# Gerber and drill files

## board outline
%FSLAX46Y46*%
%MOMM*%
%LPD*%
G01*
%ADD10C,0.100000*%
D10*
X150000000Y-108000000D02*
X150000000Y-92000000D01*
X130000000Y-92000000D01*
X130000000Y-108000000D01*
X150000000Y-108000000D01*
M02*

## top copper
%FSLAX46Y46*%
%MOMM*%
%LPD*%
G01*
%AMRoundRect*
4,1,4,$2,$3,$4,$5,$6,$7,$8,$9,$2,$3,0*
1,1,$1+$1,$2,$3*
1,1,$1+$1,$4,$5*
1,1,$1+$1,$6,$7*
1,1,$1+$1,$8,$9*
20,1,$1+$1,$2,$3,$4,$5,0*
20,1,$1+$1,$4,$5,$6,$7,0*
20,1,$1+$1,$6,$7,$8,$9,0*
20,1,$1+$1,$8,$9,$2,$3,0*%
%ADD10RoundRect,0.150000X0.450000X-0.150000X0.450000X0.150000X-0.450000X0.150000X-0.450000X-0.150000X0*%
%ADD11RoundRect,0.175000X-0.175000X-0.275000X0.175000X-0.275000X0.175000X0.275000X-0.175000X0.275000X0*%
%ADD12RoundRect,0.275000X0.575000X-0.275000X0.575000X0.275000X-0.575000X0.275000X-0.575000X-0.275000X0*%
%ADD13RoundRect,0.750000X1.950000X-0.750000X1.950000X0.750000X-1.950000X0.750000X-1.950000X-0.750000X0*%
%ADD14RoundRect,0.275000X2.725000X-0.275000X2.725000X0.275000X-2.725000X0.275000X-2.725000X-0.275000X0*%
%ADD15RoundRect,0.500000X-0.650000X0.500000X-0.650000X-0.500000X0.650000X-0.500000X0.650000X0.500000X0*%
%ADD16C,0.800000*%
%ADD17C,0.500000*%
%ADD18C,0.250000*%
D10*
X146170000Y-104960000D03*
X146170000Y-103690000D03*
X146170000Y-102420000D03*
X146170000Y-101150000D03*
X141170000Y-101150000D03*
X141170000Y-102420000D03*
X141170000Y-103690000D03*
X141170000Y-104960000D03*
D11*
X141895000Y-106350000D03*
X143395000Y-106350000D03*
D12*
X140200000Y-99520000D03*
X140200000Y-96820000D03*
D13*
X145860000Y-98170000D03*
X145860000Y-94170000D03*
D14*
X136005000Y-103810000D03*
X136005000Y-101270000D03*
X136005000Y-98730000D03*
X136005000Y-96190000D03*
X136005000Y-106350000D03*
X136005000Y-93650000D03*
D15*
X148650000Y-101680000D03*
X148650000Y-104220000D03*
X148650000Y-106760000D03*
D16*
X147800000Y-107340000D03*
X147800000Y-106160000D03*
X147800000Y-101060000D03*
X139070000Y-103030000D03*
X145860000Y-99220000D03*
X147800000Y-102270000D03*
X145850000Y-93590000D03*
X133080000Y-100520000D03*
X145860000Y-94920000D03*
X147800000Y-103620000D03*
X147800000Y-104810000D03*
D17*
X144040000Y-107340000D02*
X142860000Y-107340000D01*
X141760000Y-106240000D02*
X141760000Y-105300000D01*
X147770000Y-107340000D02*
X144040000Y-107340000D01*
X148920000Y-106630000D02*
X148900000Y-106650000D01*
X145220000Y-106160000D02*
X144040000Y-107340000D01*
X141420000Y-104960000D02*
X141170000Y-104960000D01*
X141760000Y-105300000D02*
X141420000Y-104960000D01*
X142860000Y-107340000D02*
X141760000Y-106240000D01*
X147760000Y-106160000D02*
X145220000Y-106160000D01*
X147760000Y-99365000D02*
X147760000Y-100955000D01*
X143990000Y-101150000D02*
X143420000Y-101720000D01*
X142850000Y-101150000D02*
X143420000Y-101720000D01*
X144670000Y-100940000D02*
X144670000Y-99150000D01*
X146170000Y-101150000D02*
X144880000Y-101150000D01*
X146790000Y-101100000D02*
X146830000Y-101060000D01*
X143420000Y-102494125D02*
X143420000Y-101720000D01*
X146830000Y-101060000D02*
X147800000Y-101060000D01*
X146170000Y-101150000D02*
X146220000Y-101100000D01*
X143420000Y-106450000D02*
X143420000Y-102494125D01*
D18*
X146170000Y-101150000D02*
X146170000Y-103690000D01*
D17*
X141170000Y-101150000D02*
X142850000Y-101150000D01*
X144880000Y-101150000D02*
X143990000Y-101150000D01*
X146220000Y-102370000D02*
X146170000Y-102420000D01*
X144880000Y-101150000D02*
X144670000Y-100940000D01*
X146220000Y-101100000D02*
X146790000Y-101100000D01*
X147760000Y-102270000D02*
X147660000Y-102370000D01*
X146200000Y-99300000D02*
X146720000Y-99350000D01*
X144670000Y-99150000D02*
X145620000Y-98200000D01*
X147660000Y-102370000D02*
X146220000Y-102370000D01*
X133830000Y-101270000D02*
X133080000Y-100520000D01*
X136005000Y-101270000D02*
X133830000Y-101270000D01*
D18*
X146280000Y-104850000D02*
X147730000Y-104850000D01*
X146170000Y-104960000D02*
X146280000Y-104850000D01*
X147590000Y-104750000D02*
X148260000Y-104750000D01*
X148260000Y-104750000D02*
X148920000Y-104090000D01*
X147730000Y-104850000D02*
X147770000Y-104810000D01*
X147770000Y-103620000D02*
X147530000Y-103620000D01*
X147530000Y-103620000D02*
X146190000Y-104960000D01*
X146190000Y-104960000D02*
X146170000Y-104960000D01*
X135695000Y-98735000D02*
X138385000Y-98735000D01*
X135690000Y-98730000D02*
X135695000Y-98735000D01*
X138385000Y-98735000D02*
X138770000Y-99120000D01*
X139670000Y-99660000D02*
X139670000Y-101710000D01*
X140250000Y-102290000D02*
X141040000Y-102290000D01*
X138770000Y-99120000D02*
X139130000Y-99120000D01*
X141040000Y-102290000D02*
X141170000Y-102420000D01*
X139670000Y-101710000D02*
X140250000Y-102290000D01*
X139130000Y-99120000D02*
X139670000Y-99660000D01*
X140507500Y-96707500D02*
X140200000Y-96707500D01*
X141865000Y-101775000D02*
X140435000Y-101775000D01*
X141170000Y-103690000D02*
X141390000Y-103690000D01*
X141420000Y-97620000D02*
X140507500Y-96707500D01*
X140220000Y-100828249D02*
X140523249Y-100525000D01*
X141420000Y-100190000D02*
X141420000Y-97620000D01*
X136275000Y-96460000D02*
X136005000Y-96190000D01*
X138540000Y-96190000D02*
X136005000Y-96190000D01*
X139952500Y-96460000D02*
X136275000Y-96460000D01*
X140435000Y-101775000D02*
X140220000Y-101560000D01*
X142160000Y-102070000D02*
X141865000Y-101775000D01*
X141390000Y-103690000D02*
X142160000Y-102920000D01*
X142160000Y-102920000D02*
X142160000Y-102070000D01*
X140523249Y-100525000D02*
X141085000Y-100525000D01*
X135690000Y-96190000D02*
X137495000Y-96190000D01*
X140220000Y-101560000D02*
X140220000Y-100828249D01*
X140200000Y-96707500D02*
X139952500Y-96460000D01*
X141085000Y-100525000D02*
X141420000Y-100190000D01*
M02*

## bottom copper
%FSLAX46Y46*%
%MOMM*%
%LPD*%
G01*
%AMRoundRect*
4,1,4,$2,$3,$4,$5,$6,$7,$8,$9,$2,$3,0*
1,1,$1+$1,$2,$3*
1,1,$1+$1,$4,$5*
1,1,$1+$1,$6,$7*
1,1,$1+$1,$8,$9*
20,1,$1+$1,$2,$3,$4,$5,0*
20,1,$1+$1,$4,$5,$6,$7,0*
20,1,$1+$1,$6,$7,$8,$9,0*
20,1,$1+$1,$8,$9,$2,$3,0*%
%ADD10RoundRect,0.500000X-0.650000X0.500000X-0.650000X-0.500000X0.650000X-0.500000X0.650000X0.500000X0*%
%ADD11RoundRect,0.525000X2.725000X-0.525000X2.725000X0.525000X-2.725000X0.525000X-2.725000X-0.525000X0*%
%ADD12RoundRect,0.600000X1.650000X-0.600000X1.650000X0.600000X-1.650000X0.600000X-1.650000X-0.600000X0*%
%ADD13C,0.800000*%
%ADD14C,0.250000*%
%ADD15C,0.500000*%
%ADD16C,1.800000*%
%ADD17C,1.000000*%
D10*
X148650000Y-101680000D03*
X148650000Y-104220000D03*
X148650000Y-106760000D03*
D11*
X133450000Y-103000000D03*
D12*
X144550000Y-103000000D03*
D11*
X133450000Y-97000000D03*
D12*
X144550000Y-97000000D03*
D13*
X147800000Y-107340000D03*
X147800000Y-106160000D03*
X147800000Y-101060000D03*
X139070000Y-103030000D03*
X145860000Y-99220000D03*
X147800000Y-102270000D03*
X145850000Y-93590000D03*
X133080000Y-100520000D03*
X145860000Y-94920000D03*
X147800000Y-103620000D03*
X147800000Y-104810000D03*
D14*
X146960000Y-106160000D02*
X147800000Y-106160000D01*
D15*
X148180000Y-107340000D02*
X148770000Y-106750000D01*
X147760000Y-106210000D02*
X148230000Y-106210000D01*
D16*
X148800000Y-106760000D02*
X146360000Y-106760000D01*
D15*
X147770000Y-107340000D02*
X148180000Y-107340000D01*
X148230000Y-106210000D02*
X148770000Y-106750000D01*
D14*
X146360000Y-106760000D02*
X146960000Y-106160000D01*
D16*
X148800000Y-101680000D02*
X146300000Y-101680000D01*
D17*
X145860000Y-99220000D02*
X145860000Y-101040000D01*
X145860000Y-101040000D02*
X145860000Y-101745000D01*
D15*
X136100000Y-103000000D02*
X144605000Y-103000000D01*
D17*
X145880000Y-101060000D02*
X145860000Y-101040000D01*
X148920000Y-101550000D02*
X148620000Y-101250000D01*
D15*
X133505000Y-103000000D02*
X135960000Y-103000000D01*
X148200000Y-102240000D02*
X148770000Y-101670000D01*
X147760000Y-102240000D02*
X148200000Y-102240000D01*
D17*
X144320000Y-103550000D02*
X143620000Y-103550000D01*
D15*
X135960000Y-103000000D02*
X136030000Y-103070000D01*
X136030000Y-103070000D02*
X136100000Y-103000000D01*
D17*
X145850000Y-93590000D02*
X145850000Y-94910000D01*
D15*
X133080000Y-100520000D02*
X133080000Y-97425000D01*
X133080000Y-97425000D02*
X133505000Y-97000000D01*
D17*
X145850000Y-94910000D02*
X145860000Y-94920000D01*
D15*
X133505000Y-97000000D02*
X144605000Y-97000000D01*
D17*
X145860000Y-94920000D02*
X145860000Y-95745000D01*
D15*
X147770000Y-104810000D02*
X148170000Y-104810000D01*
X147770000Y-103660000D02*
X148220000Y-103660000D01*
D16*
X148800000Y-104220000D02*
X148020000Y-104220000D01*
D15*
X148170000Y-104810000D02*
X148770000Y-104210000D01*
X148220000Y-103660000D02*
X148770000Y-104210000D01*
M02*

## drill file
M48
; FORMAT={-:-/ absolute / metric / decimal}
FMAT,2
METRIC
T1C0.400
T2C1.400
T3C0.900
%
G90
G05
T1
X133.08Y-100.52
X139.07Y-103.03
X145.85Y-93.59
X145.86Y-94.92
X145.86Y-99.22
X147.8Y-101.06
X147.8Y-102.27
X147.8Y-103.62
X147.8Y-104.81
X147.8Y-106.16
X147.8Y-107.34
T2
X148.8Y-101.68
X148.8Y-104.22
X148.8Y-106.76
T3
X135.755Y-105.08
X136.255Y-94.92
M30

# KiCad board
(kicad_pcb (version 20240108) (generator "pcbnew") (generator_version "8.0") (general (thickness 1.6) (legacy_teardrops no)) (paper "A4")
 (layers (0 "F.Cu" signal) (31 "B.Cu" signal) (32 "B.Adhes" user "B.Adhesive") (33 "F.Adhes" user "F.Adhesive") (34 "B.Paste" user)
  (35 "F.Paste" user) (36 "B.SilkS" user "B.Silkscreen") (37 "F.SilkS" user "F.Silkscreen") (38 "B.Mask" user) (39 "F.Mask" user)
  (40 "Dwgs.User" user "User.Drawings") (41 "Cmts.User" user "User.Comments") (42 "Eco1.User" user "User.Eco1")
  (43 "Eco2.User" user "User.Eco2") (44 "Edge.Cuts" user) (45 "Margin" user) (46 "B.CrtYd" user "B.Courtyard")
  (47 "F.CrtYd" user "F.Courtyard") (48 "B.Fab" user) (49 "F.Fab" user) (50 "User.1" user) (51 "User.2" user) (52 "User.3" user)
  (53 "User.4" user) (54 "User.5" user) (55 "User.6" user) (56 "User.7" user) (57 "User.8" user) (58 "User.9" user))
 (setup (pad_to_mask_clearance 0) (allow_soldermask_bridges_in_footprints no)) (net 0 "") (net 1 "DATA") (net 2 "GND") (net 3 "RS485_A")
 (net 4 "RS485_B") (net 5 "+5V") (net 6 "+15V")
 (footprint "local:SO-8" (layer "F.Cu") (at 143.67 103.055 90)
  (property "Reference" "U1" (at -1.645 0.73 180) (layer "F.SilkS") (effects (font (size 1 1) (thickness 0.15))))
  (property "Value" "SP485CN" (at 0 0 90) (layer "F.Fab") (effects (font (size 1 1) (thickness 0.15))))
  (pad "1" smd roundrect (at -1.905 2.5 90) (size 0.6 1.2) (layers "F.Cu" "F.Paste" "F.Mask") (roundrect_rratio 0.25) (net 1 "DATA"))
  (pad "2" smd roundrect (at -0.635 2.5 90) (size 0.6 1.2) (layers "F.Cu" "F.Paste" "F.Mask") (roundrect_rratio 0.25) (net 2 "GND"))
  (pad "3" smd roundrect (at 0.635 2.5 90) (size 0.6 1.2) (layers "F.Cu" "F.Paste" "F.Mask") (roundrect_rratio 0.25) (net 2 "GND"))
  (pad "4" smd roundrect (at 1.905 2.5 90) (size 0.6 1.2) (layers "F.Cu" "F.Paste" "F.Mask") (roundrect_rratio 0.25) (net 2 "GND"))
  (pad "5" smd roundrect (at 1.905 -2.5 90) (size 0.6 1.2) (layers "F.Cu" "F.Paste" "F.Mask") (roundrect_rratio 0.25) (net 2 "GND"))
  (pad "6" smd roundrect (at 0.635 -2.5 90) (size 0.6 1.2) (layers "F.Cu" "F.Paste" "F.Mask") (roundrect_rratio 0.25) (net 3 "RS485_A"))
  (pad "7" smd roundrect (at -0.635 -2.5 90) (size 0.6 1.2) (layers "F.Cu" "F.Paste" "F.Mask") (roundrect_rratio 0.25) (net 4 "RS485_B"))
  (pad "8" smd roundrect (at -1.905 -2.5 90) (size 0.6 1.2) (layers "F.Cu" "F.Paste" "F.Mask") (roundrect_rratio 0.25) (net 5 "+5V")))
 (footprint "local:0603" (layer "F.Cu") (at 142.645 106.35)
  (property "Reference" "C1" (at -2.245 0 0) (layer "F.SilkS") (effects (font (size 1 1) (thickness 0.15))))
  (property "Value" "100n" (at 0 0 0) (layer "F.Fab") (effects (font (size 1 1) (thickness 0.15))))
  (pad "1" smd roundrect (at -0.75 0) (size 0.7 0.9) (layers "F.Cu" "F.Paste" "F.Mask") (roundrect_rratio 0.25) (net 5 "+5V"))
  (pad "2" smd roundrect (at 0.75 0) (size 0.7 0.9) (layers "F.Cu" "F.Paste" "F.Mask") (roundrect_rratio 0.25) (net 2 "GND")))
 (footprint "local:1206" (layer "F.Cu") (at 140.2 98.17 90)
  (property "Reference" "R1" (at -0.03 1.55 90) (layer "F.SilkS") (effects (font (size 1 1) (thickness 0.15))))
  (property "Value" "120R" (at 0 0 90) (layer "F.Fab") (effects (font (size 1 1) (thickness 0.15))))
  (pad "1" smd roundrect (at -1.35 0 90) (size 1.1 1.7) (layers "F.Cu" "F.Paste" "F.Mask") (roundrect_rratio 0.25) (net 3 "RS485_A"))
  (pad "2" smd roundrect (at 1.35 0 90) (size 1.1 1.7) (layers "F.Cu" "F.Paste" "F.Mask") (roundrect_rratio 0.25) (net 4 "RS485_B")))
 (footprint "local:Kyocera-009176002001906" (layer "F.Cu") (at 145.86 96.17 90)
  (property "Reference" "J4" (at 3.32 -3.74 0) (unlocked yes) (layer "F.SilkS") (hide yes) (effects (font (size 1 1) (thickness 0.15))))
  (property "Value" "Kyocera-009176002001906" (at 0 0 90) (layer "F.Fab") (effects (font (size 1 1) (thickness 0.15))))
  (pad "1" smd roundrect (at -2 0 90) (size 3 5.4) (layers "F.Cu" "F.Paste" "F.Mask") (roundrect_rratio 0.25) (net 2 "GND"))
  (pad "2" smd roundrect (at 2 0 90) (size 3 5.4) (layers "F.Cu" "F.Paste" "F.Mask") (roundrect_rratio 0.25) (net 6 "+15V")))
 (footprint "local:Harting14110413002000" (layer "F.Cu") (at 136.005 100 90)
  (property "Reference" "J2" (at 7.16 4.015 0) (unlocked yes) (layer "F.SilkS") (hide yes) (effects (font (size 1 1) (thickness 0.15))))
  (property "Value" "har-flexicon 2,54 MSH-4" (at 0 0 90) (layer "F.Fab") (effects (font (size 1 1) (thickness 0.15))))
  (pad "" np_thru_hole circle (at -5.08 -0.25 90) (size 0.9 0.9) (drill 0.9) (layers "*.Cu" "*.Mask"))
  (pad "" np_thru_hole circle (at 5.08 0.25 90) (size 0.9 0.9) (drill 0.9) (layers "*.Cu" "*.Mask"))
  (pad "1" smd roundrect (at -3.81 0 90) (size 1.1 6) (layers "F.Cu" "F.Paste" "F.Mask") (roundrect_rratio 0.25) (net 2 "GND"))
  (pad "2" smd roundrect (at -1.27 0 90) (size 1.1 6) (layers "F.Cu" "F.Paste" "F.Mask") (roundrect_rratio 0.25) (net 6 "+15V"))
  (pad "3" smd roundrect (at 1.27 0 90) (size 1.1 6) (layers "F.Cu" "F.Paste" "F.Mask") (roundrect_rratio 0.25) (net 3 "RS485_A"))
  (pad "4" smd roundrect (at 3.81 0 90) (size 1.1 6) (layers "F.Cu" "F.Paste" "F.Mask") (roundrect_rratio 0.25) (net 4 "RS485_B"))
  (pad "MP1" smd roundrect (at -6.35 0 90) (size 1.1 6) (layers "F.Cu" "F.Paste" "F.Mask") (roundrect_rratio 0.25))
  (pad "MP2" smd roundrect (at 6.35 0 90) (size 1.1 6) (layers "F.Cu" "F.Paste" "F.Mask") (roundrect_rratio 0.25)))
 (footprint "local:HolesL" (layer "F.Cu") (at 148.8 104.22 -90)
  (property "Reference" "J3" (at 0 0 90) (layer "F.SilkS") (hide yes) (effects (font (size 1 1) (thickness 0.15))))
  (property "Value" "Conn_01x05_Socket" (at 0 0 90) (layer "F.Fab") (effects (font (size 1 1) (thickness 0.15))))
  (pad "1" thru_hole roundrect (at -2.54 0 270) (size 2 2.3) (drill 1.4 (offset 0 0.15)) (layers "*.Cu" "*.Mask") (remove_unused_layers yes)
   (keep_end_layers yes) (zone_layer_connections) (roundrect_rratio 0.25) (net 2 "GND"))
  (pad "2" thru_hole roundrect (at 0 0 270) (size 2 2.3) (drill 1.4 (offset 0 0.15)) (layers "*.Cu" "*.Mask") (remove_unused_layers yes)
   (keep_end_layers yes) (zone_layer_connections) (roundrect_rratio 0.25) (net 1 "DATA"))
  (pad "3" thru_hole roundrect (at 2.54 0 270) (size 2 2.3) (drill 1.4 (offset 0 0.15)) (layers "*.Cu" "*.Mask") (remove_unused_layers yes)
   (keep_end_layers yes) (zone_layer_connections) (roundrect_rratio 0.25) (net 5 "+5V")))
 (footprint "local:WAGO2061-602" (layer "B.Cu") (at 138.2 100 90)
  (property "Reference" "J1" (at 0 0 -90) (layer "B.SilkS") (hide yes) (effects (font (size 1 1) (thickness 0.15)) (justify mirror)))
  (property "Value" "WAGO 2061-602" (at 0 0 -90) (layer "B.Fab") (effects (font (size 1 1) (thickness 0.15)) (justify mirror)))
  (pad "1" smd roundrect (at -3 -4.75 90) (size 2.1 6.5) (layers "B.Cu" "B.Paste" "B.Mask") (roundrect_rratio 0.25) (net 2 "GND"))
  (pad "1" smd roundrect (at -3 6.35 90) (size 2.4 4.5) (layers "B.Cu" "B.Paste" "B.Mask") (roundrect_rratio 0.25) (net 2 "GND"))
  (pad "2" smd roundrect (at 3 -4.75 90) (size 2.1 6.5) (layers "B.Cu" "B.Paste" "B.Mask") (roundrect_rratio 0.25) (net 6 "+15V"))
  (pad "2" smd roundrect (at 3 6.35 90) (size 2.4 4.5) (layers "B.Cu" "B.Paste" "B.Mask") (roundrect_rratio 0.25) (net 6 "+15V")))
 (gr_poly (pts (xy 150 108) (xy 150 92) (xy 130 92) (xy 130 108)) (stroke (width 0.1) (type solid)) (fill none) (layer "Edge.Cuts"))
 (segment (start 144.04 107.34) (end 142.86 107.34) (width 0.5) (layer "F.Cu") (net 5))
 (segment (start 141.76 106.24) (end 141.76 105.3) (width 0.5) (layer "F.Cu") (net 5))
 (segment (start 147.77 107.34) (end 144.04 107.34) (width 0.5) (layer "F.Cu") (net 5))
 (segment (start 148.92 106.63) (end 148.9 106.65) (width 0.5) (layer "F.Cu") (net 5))
 (segment (start 145.22 106.16) (end 144.04 107.34) (width 0.5) (layer "F.Cu") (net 5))
 (segment (start 141.42 104.96) (end 141.17 104.96) (width 0.5) (layer "F.Cu") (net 5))
 (segment (start 141.76 105.3) (end 141.42 104.96) (width 0.5) (layer "F.Cu") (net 5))
 (segment (start 142.86 107.34) (end 141.76 106.24) (width 0.5) (layer "F.Cu") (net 5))
 (segment (start 147.76 106.16) (end 145.22 106.16) (width 0.5) (layer "F.Cu") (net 5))
 (via (at 147.8 107.34) (size 0.8) (drill 0.4) (layers "F.Cu" "B.Cu") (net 5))
 (via (at 147.8 106.16) (size 0.8) (drill 0.4) (layers "F.Cu" "B.Cu") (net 5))
 (segment (start 146.96 106.16) (end 147.8 106.16) (width 0.25) (layer "B.Cu") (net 5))
 (segment (start 148.18 107.34) (end 148.77 106.75) (width 0.5) (layer "B.Cu") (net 5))
 (segment (start 147.76 106.21) (end 148.23 106.21) (width 0.5) (layer "B.Cu") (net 5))
 (segment (start 148.8 106.76) (end 146.36 106.76) (width 1.8) (layer "B.Cu") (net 5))
 (segment (start 147.77 107.34) (end 148.18 107.34) (width 0.5) (layer "B.Cu") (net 5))
 (segment (start 148.23 106.21) (end 148.77 106.75) (width 0.5) (layer "B.Cu") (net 5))
 (segment (start 146.36 106.76) (end 146.96 106.16) (width 0.25) (layer "B.Cu") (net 5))
 (segment (start 147.76 99.365) (end 147.76 100.955) (width 0.5) (layer "F.Cu") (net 2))
 (segment (start 143.99 101.15) (end 143.42 101.72) (width 0.5) (layer "F.Cu") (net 2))
 (segment (start 142.85 101.15) (end 143.42 101.72) (width 0.5) (layer "F.Cu") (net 2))
 (segment (start 144.67 100.94) (end 144.67 99.15) (width 0.5) (layer "F.Cu") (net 2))
 (segment (start 146.17 101.15) (end 144.88 101.15) (width 0.5) (layer "F.Cu") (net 2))
 (segment (start 146.79 101.1) (end 146.83 101.06) (width 0.5) (layer "F.Cu") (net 2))
 (segment (start 143.42 102.494125) (end 143.42 101.72) (width 0.5) (layer "F.Cu") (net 2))
 (segment (start 146.83 101.06) (end 147.8 101.06) (width 0.5) (layer "F.Cu") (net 2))
 (segment (start 146.17 101.15) (end 146.22 101.1) (width 0.5) (layer "F.Cu") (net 2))
 (segment (start 143.42 106.45) (end 143.42 102.494125) (width 0.5) (layer "F.Cu") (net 2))
 (segment (start 146.17 101.15) (end 146.17 103.69) (width 0.25) (layer "F.Cu") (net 2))
 (segment (start 141.17 101.15) (end 142.85 101.15) (width 0.5) (layer "F.Cu") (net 2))
 (segment (start 144.88 101.15) (end 143.99 101.15) (width 0.5) (layer "F.Cu") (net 2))
 (segment (start 146.22 102.37) (end 146.17 102.42) (width 0.5) (layer "F.Cu") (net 2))
 (segment (start 144.88 101.15) (end 144.67 100.94) (width 0.5) (layer "F.Cu") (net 2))
 (segment (start 146.22 101.1) (end 146.79 101.1) (width 0.5) (layer "F.Cu") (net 2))
 (segment (start 147.76 102.27) (end 147.66 102.37) (width 0.5) (layer "F.Cu") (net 2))
 (segment (start 146.2 99.3) (end 146.72 99.35) (width 0.5) (layer "F.Cu") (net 2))
 (segment (start 144.67 99.15) (end 145.62 98.2) (width 0.5) (layer "F.Cu") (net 2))
 (segment (start 147.66 102.37) (end 146.22 102.37) (width 0.5) (layer "F.Cu") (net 2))
 (via (at 147.8 101.06) (size 0.8) (drill 0.4) (layers "F.Cu" "B.Cu") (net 2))
 (via (at 139.07 103.03) (size 0.8) (drill 0.4) (layers "F.Cu" "B.Cu") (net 2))
 (via (at 145.86 99.22) (size 0.8) (drill 0.4) (layers "F.Cu" "B.Cu") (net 2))
 (via (at 147.8 102.27) (size 0.8) (drill 0.4) (layers "F.Cu" "B.Cu") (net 2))
 (segment (start 148.8 101.68) (end 146.3 101.68) (width 1.8) (layer "B.Cu") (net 2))
 (segment (start 145.86 99.22) (end 145.86 101.04) (width 1) (layer "B.Cu") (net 2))
 (segment (start 145.86 101.04) (end 145.86 101.745) (width 1) (layer "B.Cu") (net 2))
 (segment (start 136.1 103) (end 144.605 103) (width 0.5) (layer "B.Cu") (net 2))
 (segment (start 145.88 101.06) (end 145.86 101.04) (width 1) (layer "B.Cu") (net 2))
 (segment (start 148.92 101.55) (end 148.62 101.25) (width 1) (layer "B.Cu") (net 2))
 (segment (start 133.505 103) (end 135.96 103) (width 0.5) (layer "B.Cu") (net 2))
 (segment (start 148.2 102.24) (end 148.77 101.67) (width 0.5) (layer "B.Cu") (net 2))
 (segment (start 147.76 102.24) (end 148.2 102.24) (width 0.5) (layer "B.Cu") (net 2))
 (segment (start 144.32 103.55) (end 143.62 103.55) (width 1) (layer "B.Cu") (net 2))
 (segment (start 135.96 103) (end 136.03 103.07) (width 0.5) (layer "B.Cu") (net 2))
 (segment (start 136.03 103.07) (end 136.1 103) (width 0.5) (layer "B.Cu") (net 2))
 (segment (start 133.83 101.27) (end 133.08 100.52) (width 0.5) (layer "F.Cu") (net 6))
 (segment (start 136.005 101.27) (end 133.83 101.27) (width 0.5) (layer "F.Cu") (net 6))
 (via (at 145.85 93.59) (size 0.8) (drill 0.4) (layers "F.Cu" "B.Cu") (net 6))
 (via (at 133.08 100.52) (size 0.8) (drill 0.4) (layers "F.Cu" "B.Cu") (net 6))
 (via (at 145.86 94.92) (size 0.8) (drill 0.4) (layers "F.Cu" "B.Cu") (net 6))
 (segment (start 145.85 93.59) (end 145.85 94.91) (width 1) (layer "B.Cu") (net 6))
 (segment (start 133.08 100.52) (end 133.08 97.425) (width 0.5) (layer "B.Cu") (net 6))
 (segment (start 133.08 97.425) (end 133.505 97) (width 0.5) (layer "B.Cu") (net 6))
 (segment (start 145.85 94.91) (end 145.86 94.92) (width 1) (layer "B.Cu") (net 6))
 (segment (start 133.505 97) (end 144.605 97) (width 0.5) (layer "B.Cu") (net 6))
 (segment (start 145.86 94.92) (end 145.86 95.745) (width 1) (layer "B.Cu") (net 6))
 (segment (start 146.28 104.85) (end 147.73 104.85) (width 0.25) (layer "F.Cu") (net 1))
 (segment (start 146.17 104.96) (end 146.28 104.85) (width 0.25) (layer "F.Cu") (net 1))
 (segment (start 147.59 104.75) (end 148.26 104.75) (width 0.25) (layer "F.Cu") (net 1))
 (segment (start 148.26 104.75) (end 148.92 104.09) (width 0.25) (layer "F.Cu") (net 1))
 (segment (start 147.73 104.85) (end 147.77 104.81) (width 0.25) (layer "F.Cu") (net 1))
 (segment (start 147.77 103.62) (end 147.53 103.62) (width 0.25) (layer "F.Cu") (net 1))
 (segment (start 147.53 103.62) (end 146.19 104.96) (width 0.25) (layer "F.Cu") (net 1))
 (segment (start 146.19 104.96) (end 146.17 104.96) (width 0.25) (layer "F.Cu") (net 1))
 (via (at 147.8 103.62) (size 0.8) (drill 0.4) (layers "F.Cu" "B.Cu") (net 1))
 (via (at 147.8 104.81) (size 0.8) (drill 0.4) (layers "F.Cu" "B.Cu") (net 1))
 (segment (start 147.77 104.81) (end 148.17 104.81) (width 0.5) (layer "B.Cu") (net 1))
 (segment (start 147.77 103.66) (end 148.22 103.66) (width 0.5) (layer "B.Cu") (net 1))
 (segment (start 148.8 104.22) (end 148.02 104.22) (width 1.8) (layer "B.Cu") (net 1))
 (segment (start 148.17 104.81) (end 148.77 104.21) (width 0.5) (layer "B.Cu") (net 1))
 (segment (start 148.22 103.66) (end 148.77 104.21) (width 0.5) (layer "B.Cu") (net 1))
 (segment (start 135.695 98.735) (end 138.385 98.735) (width 0.25) (layer "F.Cu") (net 3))
 (segment (start 135.69 98.73) (end 135.695 98.735) (width 0.25) (layer "F.Cu") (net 3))
 (segment (start 138.385 98.735) (end 138.77 99.12) (width 0.25) (layer "F.Cu") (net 3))
 (segment (start 139.67 99.66) (end 139.67 101.71) (width 0.25) (layer "F.Cu") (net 3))
 (segment (start 140.25 102.29) (end 141.04 102.29) (width 0.25) (layer "F.Cu") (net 3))
 (segment (start 138.77 99.12) (end 139.13 99.12) (width 0.25) (layer "F.Cu") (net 3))
 (segment (start 141.04 102.29) (end 141.17 102.42) (width 0.25) (layer "F.Cu") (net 3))
 (segment (start 139.67 101.71) (end 140.25 102.29) (width 0.25) (layer "F.Cu") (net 3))
 (segment (start 139.13 99.12) (end 139.67 99.66) (width 0.25) (layer "F.Cu") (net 3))
 (segment (start 140.5075 96.7075) (end 140.2 96.7075) (width 0.25) (layer "F.Cu") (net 4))
 (segment (start 141.865 101.775) (end 140.435 101.775) (width 0.25) (layer "F.Cu") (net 4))
 (segment (start 141.17 103.69) (end 141.39 103.69) (width 0.25) (layer "F.Cu") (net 4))
 (segment (start 141.42 97.62) (end 140.5075 96.7075) (width 0.25) (layer "F.Cu") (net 4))
 (segment (start 140.22 100.828249) (end 140.523249 100.525) (width 0.25) (layer "F.Cu") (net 4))
 (segment (start 141.42 100.19) (end 141.42 97.62) (width 0.25) (layer "F.Cu") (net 4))
 (segment (start 136.275 96.46) (end 136.005 96.19) (width 0.25) (layer "F.Cu") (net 4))
 (segment (start 138.54 96.19) (end 136.005 96.19) (width 0.25) (layer "F.Cu") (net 4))
 (segment (start 139.9525 96.46) (end 136.275 96.46) (width 0.25) (layer "F.Cu") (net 4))
 (segment (start 140.435 101.775) (end 140.22 101.56) (width 0.25) (layer "F.Cu") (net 4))
 (segment (start 142.16 102.07) (end 141.865 101.775) (width 0.25) (layer "F.Cu") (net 4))
 (segment (start 141.39 103.69) (end 142.16 102.92) (width 0.25) (layer "F.Cu") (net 4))
 (segment (start 142.16 102.92) (end 142.16 102.07) (width 0.25) (layer "F.Cu") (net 4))
 (segment (start 140.523249 100.525) (end 141.085 100.525) (width 0.25) (layer "F.Cu") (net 4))
 (segment (start 135.69 96.19) (end 137.495 96.19) (width 0.25) (layer "F.Cu") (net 4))
 (segment (start 140.22 101.56) (end 140.22 100.828249) (width 0.25) (layer "F.Cu") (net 4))
 (segment (start 140.2 96.7075) (end 139.9525 96.46) (width 0.25) (layer "F.Cu") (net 4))
 (segment (start 141.085 100.525) (end 141.42 100.19) (width 0.25) (layer "F.Cu") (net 4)))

